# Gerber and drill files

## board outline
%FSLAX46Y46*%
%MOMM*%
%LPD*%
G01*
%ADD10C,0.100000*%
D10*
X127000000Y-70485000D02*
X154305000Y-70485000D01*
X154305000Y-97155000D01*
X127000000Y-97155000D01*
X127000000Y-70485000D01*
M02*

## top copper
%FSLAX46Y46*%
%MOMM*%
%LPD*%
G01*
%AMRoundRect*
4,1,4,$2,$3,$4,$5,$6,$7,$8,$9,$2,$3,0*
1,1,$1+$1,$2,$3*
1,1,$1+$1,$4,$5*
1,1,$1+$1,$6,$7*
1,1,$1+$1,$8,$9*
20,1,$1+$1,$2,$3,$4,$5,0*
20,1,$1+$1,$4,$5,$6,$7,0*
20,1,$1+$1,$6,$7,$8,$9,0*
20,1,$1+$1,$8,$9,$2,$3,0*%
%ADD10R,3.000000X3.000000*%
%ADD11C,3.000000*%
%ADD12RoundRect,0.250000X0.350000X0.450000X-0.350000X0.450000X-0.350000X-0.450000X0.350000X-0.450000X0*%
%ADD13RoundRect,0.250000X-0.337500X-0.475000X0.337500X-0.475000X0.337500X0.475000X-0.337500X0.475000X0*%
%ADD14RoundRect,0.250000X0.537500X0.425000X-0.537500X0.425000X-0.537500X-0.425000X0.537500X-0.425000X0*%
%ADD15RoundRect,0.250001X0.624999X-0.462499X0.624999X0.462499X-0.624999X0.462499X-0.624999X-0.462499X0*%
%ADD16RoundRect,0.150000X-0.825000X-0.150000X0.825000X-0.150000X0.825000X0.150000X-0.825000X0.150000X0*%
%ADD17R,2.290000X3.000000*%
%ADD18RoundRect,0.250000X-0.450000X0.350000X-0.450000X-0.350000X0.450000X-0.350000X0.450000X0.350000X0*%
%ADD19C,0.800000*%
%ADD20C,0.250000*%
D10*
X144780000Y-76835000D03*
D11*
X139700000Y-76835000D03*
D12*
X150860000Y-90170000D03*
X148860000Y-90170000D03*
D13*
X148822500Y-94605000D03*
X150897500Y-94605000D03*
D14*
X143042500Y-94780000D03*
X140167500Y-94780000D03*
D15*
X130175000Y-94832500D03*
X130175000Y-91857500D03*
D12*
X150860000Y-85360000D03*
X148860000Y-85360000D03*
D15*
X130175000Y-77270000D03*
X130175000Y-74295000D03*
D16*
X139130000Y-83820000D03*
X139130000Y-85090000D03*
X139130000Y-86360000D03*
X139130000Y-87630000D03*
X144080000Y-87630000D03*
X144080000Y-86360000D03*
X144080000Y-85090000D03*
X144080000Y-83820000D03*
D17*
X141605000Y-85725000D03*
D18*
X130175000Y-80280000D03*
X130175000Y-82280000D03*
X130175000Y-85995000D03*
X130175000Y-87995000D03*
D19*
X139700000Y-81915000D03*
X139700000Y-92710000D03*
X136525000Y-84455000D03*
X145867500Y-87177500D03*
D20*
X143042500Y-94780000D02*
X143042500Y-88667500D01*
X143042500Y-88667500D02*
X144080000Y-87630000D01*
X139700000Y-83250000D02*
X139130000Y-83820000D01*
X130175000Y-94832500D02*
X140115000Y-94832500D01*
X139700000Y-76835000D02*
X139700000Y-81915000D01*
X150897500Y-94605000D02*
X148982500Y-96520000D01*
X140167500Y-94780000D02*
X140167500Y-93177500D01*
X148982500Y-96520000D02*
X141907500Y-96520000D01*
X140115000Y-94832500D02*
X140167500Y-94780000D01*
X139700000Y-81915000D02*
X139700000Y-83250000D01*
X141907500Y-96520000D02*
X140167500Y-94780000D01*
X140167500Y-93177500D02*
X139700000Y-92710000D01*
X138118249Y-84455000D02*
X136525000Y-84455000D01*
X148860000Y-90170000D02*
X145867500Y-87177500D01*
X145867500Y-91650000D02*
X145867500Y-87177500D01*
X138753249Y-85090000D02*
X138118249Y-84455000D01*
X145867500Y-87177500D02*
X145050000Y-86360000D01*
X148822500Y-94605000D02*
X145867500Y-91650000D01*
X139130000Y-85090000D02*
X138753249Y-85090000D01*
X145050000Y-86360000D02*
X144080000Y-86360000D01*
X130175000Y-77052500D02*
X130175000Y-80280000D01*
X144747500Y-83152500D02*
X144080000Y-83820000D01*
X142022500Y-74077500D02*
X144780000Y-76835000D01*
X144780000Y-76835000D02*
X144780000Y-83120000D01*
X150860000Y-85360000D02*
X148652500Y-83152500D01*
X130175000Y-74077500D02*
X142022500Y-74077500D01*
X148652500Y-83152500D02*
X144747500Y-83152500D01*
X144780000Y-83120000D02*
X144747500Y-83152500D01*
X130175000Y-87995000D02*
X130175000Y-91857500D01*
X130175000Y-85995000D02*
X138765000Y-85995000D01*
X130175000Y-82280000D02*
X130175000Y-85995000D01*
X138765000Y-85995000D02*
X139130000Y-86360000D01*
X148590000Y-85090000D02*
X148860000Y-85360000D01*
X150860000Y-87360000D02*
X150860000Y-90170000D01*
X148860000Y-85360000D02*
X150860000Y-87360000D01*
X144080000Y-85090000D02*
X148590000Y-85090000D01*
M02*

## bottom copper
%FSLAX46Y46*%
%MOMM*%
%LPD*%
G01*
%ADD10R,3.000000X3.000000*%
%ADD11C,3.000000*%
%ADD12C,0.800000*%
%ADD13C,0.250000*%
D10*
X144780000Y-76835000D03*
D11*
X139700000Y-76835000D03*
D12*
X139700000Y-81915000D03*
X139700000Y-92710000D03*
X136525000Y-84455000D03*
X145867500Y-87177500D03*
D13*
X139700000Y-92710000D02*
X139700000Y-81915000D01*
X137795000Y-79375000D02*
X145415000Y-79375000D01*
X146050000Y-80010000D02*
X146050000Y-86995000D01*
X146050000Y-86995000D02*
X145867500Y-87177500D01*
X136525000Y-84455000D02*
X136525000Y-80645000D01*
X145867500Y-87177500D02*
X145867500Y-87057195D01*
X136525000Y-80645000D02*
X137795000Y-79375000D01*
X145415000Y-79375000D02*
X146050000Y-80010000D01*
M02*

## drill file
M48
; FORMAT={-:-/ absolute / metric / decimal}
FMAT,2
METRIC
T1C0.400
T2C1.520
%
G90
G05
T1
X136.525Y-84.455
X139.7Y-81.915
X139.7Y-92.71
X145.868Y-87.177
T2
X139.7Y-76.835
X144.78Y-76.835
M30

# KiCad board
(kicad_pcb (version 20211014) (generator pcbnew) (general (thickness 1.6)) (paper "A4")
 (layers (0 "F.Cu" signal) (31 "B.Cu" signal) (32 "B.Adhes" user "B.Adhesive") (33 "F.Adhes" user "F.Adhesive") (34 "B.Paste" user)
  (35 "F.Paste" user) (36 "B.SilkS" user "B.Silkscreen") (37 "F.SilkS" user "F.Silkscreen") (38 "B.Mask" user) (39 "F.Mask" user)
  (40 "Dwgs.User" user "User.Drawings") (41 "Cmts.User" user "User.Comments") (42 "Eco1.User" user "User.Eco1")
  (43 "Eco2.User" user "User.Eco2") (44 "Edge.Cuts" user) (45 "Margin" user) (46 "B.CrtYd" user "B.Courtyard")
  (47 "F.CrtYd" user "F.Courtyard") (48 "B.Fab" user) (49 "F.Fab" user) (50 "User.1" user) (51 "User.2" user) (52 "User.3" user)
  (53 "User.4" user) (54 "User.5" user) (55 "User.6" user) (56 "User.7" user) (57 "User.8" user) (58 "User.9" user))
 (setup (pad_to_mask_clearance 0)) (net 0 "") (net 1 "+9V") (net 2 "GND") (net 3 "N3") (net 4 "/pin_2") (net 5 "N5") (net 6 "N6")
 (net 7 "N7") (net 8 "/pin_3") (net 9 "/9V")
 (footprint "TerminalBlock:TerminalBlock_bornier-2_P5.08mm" (layer "F.Cu") (at 144.78 76.835 180)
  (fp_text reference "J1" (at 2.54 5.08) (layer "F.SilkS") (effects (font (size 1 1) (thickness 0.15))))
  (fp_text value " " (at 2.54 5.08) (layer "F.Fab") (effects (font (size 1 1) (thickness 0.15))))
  (pad "1" thru_hole rect (at 0 0 180) (size 3 3) (drill 1.52) (layers *.Cu *.Mask) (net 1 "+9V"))
  (pad "2" thru_hole circle (at 5.08 0 180) (size 3 3) (drill 1.52) (layers *.Cu *.Mask) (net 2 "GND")))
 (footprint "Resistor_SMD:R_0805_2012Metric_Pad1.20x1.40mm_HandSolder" (layer "F.Cu") (at 149.86 90.17 180)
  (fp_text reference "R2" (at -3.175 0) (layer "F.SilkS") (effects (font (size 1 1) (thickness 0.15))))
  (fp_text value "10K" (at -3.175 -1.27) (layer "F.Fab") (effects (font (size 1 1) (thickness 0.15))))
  (pad "1" smd roundrect (at -1 0 180) (size 1.2 1.4) (layers "F.Cu" "F.Paste" "F.Mask") (roundrect_rratio 0.208333) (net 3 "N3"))
  (pad "2" smd roundrect (at 1 0 180) (size 1.2 1.4) (layers "F.Cu" "F.Paste" "F.Mask") (roundrect_rratio 0.208333) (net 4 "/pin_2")))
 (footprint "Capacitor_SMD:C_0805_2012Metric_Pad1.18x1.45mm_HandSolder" (layer "F.Cu") (at 149.86 94.605)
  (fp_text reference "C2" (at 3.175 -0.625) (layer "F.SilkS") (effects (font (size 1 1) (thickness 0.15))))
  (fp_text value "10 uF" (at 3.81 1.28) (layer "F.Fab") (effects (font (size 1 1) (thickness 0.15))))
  (pad "2" smd roundrect (at -1.0375 0) (size 1.175 1.45) (layers "F.Cu" "F.Paste" "F.Mask") (roundrect_rratio 0.212766) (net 4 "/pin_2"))
  (pad "2" smd roundrect (at 1.0375 0) (size 1.175 1.45) (layers "F.Cu" "F.Paste" "F.Mask") (roundrect_rratio 0.212766) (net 2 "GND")))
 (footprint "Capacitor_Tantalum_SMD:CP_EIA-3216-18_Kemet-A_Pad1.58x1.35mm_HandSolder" (layer "F.Cu") (at 141.605 94.78 180)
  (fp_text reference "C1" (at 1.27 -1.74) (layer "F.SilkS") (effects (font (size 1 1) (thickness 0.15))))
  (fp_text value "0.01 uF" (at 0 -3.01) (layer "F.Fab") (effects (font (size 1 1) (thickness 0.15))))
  (pad "1" smd roundrect (at -1.4375 0 180) (size 1.575 1.35) (layers "F.Cu" "F.Paste" "F.Mask") (roundrect_rratio 0.185185) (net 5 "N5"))
  (pad "2" smd roundrect (at 1.4375 0 180) (size 1.575 1.35) (layers "F.Cu" "F.Paste" "F.Mask") (roundrect_rratio 0.185185) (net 2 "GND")))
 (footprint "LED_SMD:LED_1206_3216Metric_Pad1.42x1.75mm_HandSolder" (layer "F.Cu") (at 130.175 93.345 90)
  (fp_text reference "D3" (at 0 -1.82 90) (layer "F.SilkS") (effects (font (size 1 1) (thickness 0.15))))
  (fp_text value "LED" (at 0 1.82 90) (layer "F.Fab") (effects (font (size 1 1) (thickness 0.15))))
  (pad "1" smd roundrect (at -1.4875 0 90) (size 1.425 1.75) (layers "F.Cu" "F.Paste" "F.Mask") (roundrect_rratio 0.175439) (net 2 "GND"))
  (pad "2" smd roundrect (at 1.4875 0 90) (size 1.425 1.75) (layers "F.Cu" "F.Paste" "F.Mask") (roundrect_rratio 0.175439) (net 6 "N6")))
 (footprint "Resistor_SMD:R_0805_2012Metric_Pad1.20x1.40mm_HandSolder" (layer "F.Cu") (at 149.86 85.36 180)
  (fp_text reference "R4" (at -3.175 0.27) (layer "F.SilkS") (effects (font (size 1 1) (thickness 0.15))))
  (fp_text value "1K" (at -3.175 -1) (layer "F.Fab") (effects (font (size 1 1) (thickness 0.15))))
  (pad "1" smd roundrect (at -1 0 180) (size 1.2 1.4) (layers "F.Cu" "F.Paste" "F.Mask") (roundrect_rratio 0.208333) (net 1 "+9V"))
  (pad "2" smd roundrect (at 1 0 180) (size 1.2 1.4) (layers "F.Cu" "F.Paste" "F.Mask") (roundrect_rratio 0.208333) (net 3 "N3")))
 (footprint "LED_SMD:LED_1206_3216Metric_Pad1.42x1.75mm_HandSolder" (layer "F.Cu") (at 130.175 75.7825 90)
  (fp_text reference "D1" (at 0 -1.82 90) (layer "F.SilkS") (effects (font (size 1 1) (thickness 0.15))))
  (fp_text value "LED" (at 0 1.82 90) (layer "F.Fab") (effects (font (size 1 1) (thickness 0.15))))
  (pad "1" smd roundrect (at -1.4875 0 90) (size 1.425 1.75) (layers "F.Cu" "F.Paste" "F.Mask") (roundrect_rratio 0.175439) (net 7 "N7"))
  (pad "2" smd roundrect (at 1.4875 0 90) (size 1.425 1.75) (layers "F.Cu" "F.Paste" "F.Mask") (roundrect_rratio 0.175439) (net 1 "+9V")))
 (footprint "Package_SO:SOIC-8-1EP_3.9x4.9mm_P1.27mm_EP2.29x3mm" (layer "F.Cu") (at 141.605 85.725)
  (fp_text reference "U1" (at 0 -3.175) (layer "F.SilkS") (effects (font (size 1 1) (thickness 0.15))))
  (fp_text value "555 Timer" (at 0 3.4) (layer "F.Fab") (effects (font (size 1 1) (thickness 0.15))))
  (pad "" smd roundrect (at 0.57 -0.75) (size 0.92 1.21) (layers "F.Paste") (roundrect_rratio 0.25))
  (pad "" smd roundrect (at 0.57 0.75) (size 0.92 1.21) (layers "F.Paste") (roundrect_rratio 0.25))
  (pad "" smd roundrect (at -0.57 0.75) (size 0.92 1.21) (layers "F.Paste") (roundrect_rratio 0.25))
  (pad "" smd roundrect (at -0.57 -0.75) (size 0.92 1.21) (layers "F.Paste") (roundrect_rratio 0.25))
  (pad "1" smd roundrect (at -2.475 -1.905) (size 1.95 0.6) (layers "F.Cu" "F.Paste" "F.Mask") (roundrect_rratio 0.25) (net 2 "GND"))
  (pad "2" smd roundrect (at -2.475 -0.635) (size 1.95 0.6) (layers "F.Cu" "F.Paste" "F.Mask") (roundrect_rratio 0.25) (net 4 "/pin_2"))
  (pad "3" smd roundrect (at -2.475 0.635) (size 1.95 0.6) (layers "F.Cu" "F.Paste" "F.Mask") (roundrect_rratio 0.25) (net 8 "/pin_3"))
  (pad "4" smd roundrect (at -2.475 1.905) (size 1.95 0.6) (layers "F.Cu" "F.Paste" "F.Mask") (roundrect_rratio 0.25) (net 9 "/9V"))
  (pad "5" smd roundrect (at 2.475 1.905) (size 1.95 0.6) (layers "F.Cu" "F.Paste" "F.Mask") (roundrect_rratio 0.25) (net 5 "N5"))
  (pad "6" smd roundrect (at 2.475 0.635) (size 1.95 0.6) (layers "F.Cu" "F.Paste" "F.Mask") (roundrect_rratio 0.25) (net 4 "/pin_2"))
  (pad "7" smd roundrect (at 2.475 -0.635) (size 1.95 0.6) (layers "F.Cu" "F.Paste" "F.Mask") (roundrect_rratio 0.25) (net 3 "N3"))
  (pad "8" smd roundrect (at 2.475 -1.905) (size 1.95 0.6) (layers "F.Cu" "F.Paste" "F.Mask") (roundrect_rratio 0.25) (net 1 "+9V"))
  (pad "9" smd rect (at 0 0) (size 2.29 3) (layers "F.Cu" "F.Mask")))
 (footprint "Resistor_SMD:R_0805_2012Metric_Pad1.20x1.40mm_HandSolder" (layer "F.Cu") (at 130.175 81.28 -90)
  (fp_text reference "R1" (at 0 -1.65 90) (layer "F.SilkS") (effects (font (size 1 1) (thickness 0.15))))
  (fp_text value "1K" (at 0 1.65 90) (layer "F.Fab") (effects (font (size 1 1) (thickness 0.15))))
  (pad "1" smd roundrect (at -1 0 270) (size 1.2 1.4) (layers "F.Cu" "F.Paste" "F.Mask") (roundrect_rratio 0.208333) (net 7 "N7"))
  (pad "2" smd roundrect (at 1 0 270) (size 1.2 1.4) (layers "F.Cu" "F.Paste" "F.Mask") (roundrect_rratio 0.208333) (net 8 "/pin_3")))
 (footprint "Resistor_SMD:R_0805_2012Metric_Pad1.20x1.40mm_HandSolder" (layer "F.Cu") (at 130.175 86.995 -90)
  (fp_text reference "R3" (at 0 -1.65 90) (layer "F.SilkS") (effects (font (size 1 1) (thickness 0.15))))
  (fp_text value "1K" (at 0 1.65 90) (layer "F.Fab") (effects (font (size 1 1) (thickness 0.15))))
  (pad "1" smd roundrect (at -1 0 270) (size 1.2 1.4) (layers "F.Cu" "F.Paste" "F.Mask") (roundrect_rratio 0.208333) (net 8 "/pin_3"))
  (pad "2" smd roundrect (at 1 0 270) (size 1.2 1.4) (layers "F.Cu" "F.Paste" "F.Mask") (roundrect_rratio 0.208333) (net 6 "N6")))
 (gr_rect (start 127 70.485) (end 154.305 97.155) (layer "Edge.Cuts") (width 0.1) (fill none))
 (segment (start 143.0425 94.78) (end 143.0425 88.6675) (width 0.25) (layer "F.Cu") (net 5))
 (segment (start 143.0425 88.6675) (end 144.08 87.63) (width 0.25) (layer "F.Cu") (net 5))
 (segment (start 139.7 83.25) (end 139.13 83.82) (width 0.25) (layer "F.Cu") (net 2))
 (segment (start 130.175 94.8325) (end 140.115 94.8325) (width 0.25) (layer "F.Cu") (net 2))
 (segment (start 139.7 76.835) (end 139.7 81.915) (width 0.25) (layer "F.Cu") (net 2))
 (segment (start 150.8975 94.605) (end 148.9825 96.52) (width 0.25) (layer "F.Cu") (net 2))
 (segment (start 140.1675 94.78) (end 140.1675 93.1775) (width 0.25) (layer "F.Cu") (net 2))
 (segment (start 148.9825 96.52) (end 141.9075 96.52) (width 0.25) (layer "F.Cu") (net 2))
 (segment (start 140.115 94.8325) (end 140.1675 94.78) (width 0.25) (layer "F.Cu") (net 2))
 (segment (start 139.7 81.915) (end 139.7 83.25) (width 0.25) (layer "F.Cu") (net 2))
 (segment (start 141.9075 96.52) (end 140.1675 94.78) (width 0.25) (layer "F.Cu") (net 2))
 (segment (start 140.1675 93.1775) (end 139.7 92.71) (width 0.25) (layer "F.Cu") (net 2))
 (via (at 139.7 81.915) (size 0.8) (drill 0.4) (layers "F.Cu" "B.Cu") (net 2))
 (via (at 139.7 92.71) (size 0.8) (drill 0.4) (layers "F.Cu" "B.Cu") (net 2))
 (segment (start 139.7 92.71) (end 139.7 81.915) (width 0.25) (layer "B.Cu") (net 2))
 (segment (start 138.118249 84.455) (end 136.525 84.455) (width 0.25) (layer "F.Cu") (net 4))
 (segment (start 148.86 90.17) (end 145.8675 87.1775) (width 0.25) (layer "F.Cu") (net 4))
 (segment (start 145.8675 91.65) (end 145.8675 87.1775) (width 0.25) (layer "F.Cu") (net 4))
 (segment (start 138.753249 85.09) (end 138.118249 84.455) (width 0.25) (layer "F.Cu") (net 4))
 (segment (start 145.8675 87.1775) (end 145.05 86.36) (width 0.25) (layer "F.Cu") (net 4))
 (segment (start 148.8225 94.605) (end 145.8675 91.65) (width 0.25) (layer "F.Cu") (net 4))
 (segment (start 139.13 85.09) (end 138.753249 85.09) (width 0.25) (layer "F.Cu") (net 4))
 (segment (start 145.05 86.36) (end 144.08 86.36) (width 0.25) (layer "F.Cu") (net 4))
 (via (at 136.525 84.455) (size 0.8) (drill 0.4) (layers "F.Cu" "B.Cu") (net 4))
 (via (at 145.8675 87.1775) (size 0.8) (drill 0.4) (layers "F.Cu" "B.Cu") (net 4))
 (segment (start 137.795 79.375) (end 145.415 79.375) (width 0.25) (layer "B.Cu") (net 4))
 (segment (start 146.05 80.01) (end 146.05 86.995) (width 0.25) (layer "B.Cu") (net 4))
 (segment (start 146.05 86.995) (end 145.8675 87.1775) (width 0.25) (layer "B.Cu") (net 4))
 (segment (start 136.525 84.455) (end 136.525 80.645) (width 0.25) (layer "B.Cu") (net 4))
 (segment (start 145.8675 87.1775) (end 145.8675 87.057195) (width 0.25) (layer "B.Cu") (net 4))
 (segment (start 136.525 80.645) (end 137.795 79.375) (width 0.25) (layer "B.Cu") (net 4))
 (segment (start 145.415 79.375) (end 146.05 80.01) (width 0.25) (layer "B.Cu") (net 4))
 (segment (start 130.175 77.0525) (end 130.175 80.28) (width 0.25) (layer "F.Cu") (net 7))
 (segment (start 144.7475 83.1525) (end 144.08 83.82) (width 0.25) (layer "F.Cu") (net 1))
 (segment (start 142.0225 74.0775) (end 144.78 76.835) (width 0.25) (layer "F.Cu") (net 1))
 (segment (start 144.78 76.835) (end 144.78 83.12) (width 0.25) (layer "F.Cu") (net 1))
 (segment (start 150.86 85.36) (end 148.6525 83.1525) (width 0.25) (layer "F.Cu") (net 1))
 (segment (start 130.175 74.0775) (end 142.0225 74.0775) (width 0.25) (layer "F.Cu") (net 1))
 (segment (start 148.6525 83.1525) (end 144.7475 83.1525) (width 0.25) (layer "F.Cu") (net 1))
 (segment (start 144.78 83.12) (end 144.7475 83.1525) (width 0.25) (layer "F.Cu") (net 1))
 (segment (start 130.175 87.995) (end 130.175 91.8575) (width 0.25) (layer "F.Cu") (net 6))
 (segment (start 130.175 85.995) (end 138.765 85.995) (width 0.25) (layer "F.Cu") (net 8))
 (segment (start 130.175 82.28) (end 130.175 85.995) (width 0.25) (layer "F.Cu") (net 8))
 (segment (start 138.765 85.995) (end 139.13 86.36) (width 0.25) (layer "F.Cu") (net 8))
 (segment (start 148.59 85.09) (end 148.86 85.36) (width 0.25) (layer "F.Cu") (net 3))
 (segment (start 150.86 87.36) (end 150.86 90.17) (width 0.25) (layer "F.Cu") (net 3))
 (segment (start 148.86 85.36) (end 150.86 87.36) (width 0.25) (layer "F.Cu") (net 3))
 (segment (start 144.08 85.09) (end 148.59 85.09) (width 0.25) (layer "F.Cu") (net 3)))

